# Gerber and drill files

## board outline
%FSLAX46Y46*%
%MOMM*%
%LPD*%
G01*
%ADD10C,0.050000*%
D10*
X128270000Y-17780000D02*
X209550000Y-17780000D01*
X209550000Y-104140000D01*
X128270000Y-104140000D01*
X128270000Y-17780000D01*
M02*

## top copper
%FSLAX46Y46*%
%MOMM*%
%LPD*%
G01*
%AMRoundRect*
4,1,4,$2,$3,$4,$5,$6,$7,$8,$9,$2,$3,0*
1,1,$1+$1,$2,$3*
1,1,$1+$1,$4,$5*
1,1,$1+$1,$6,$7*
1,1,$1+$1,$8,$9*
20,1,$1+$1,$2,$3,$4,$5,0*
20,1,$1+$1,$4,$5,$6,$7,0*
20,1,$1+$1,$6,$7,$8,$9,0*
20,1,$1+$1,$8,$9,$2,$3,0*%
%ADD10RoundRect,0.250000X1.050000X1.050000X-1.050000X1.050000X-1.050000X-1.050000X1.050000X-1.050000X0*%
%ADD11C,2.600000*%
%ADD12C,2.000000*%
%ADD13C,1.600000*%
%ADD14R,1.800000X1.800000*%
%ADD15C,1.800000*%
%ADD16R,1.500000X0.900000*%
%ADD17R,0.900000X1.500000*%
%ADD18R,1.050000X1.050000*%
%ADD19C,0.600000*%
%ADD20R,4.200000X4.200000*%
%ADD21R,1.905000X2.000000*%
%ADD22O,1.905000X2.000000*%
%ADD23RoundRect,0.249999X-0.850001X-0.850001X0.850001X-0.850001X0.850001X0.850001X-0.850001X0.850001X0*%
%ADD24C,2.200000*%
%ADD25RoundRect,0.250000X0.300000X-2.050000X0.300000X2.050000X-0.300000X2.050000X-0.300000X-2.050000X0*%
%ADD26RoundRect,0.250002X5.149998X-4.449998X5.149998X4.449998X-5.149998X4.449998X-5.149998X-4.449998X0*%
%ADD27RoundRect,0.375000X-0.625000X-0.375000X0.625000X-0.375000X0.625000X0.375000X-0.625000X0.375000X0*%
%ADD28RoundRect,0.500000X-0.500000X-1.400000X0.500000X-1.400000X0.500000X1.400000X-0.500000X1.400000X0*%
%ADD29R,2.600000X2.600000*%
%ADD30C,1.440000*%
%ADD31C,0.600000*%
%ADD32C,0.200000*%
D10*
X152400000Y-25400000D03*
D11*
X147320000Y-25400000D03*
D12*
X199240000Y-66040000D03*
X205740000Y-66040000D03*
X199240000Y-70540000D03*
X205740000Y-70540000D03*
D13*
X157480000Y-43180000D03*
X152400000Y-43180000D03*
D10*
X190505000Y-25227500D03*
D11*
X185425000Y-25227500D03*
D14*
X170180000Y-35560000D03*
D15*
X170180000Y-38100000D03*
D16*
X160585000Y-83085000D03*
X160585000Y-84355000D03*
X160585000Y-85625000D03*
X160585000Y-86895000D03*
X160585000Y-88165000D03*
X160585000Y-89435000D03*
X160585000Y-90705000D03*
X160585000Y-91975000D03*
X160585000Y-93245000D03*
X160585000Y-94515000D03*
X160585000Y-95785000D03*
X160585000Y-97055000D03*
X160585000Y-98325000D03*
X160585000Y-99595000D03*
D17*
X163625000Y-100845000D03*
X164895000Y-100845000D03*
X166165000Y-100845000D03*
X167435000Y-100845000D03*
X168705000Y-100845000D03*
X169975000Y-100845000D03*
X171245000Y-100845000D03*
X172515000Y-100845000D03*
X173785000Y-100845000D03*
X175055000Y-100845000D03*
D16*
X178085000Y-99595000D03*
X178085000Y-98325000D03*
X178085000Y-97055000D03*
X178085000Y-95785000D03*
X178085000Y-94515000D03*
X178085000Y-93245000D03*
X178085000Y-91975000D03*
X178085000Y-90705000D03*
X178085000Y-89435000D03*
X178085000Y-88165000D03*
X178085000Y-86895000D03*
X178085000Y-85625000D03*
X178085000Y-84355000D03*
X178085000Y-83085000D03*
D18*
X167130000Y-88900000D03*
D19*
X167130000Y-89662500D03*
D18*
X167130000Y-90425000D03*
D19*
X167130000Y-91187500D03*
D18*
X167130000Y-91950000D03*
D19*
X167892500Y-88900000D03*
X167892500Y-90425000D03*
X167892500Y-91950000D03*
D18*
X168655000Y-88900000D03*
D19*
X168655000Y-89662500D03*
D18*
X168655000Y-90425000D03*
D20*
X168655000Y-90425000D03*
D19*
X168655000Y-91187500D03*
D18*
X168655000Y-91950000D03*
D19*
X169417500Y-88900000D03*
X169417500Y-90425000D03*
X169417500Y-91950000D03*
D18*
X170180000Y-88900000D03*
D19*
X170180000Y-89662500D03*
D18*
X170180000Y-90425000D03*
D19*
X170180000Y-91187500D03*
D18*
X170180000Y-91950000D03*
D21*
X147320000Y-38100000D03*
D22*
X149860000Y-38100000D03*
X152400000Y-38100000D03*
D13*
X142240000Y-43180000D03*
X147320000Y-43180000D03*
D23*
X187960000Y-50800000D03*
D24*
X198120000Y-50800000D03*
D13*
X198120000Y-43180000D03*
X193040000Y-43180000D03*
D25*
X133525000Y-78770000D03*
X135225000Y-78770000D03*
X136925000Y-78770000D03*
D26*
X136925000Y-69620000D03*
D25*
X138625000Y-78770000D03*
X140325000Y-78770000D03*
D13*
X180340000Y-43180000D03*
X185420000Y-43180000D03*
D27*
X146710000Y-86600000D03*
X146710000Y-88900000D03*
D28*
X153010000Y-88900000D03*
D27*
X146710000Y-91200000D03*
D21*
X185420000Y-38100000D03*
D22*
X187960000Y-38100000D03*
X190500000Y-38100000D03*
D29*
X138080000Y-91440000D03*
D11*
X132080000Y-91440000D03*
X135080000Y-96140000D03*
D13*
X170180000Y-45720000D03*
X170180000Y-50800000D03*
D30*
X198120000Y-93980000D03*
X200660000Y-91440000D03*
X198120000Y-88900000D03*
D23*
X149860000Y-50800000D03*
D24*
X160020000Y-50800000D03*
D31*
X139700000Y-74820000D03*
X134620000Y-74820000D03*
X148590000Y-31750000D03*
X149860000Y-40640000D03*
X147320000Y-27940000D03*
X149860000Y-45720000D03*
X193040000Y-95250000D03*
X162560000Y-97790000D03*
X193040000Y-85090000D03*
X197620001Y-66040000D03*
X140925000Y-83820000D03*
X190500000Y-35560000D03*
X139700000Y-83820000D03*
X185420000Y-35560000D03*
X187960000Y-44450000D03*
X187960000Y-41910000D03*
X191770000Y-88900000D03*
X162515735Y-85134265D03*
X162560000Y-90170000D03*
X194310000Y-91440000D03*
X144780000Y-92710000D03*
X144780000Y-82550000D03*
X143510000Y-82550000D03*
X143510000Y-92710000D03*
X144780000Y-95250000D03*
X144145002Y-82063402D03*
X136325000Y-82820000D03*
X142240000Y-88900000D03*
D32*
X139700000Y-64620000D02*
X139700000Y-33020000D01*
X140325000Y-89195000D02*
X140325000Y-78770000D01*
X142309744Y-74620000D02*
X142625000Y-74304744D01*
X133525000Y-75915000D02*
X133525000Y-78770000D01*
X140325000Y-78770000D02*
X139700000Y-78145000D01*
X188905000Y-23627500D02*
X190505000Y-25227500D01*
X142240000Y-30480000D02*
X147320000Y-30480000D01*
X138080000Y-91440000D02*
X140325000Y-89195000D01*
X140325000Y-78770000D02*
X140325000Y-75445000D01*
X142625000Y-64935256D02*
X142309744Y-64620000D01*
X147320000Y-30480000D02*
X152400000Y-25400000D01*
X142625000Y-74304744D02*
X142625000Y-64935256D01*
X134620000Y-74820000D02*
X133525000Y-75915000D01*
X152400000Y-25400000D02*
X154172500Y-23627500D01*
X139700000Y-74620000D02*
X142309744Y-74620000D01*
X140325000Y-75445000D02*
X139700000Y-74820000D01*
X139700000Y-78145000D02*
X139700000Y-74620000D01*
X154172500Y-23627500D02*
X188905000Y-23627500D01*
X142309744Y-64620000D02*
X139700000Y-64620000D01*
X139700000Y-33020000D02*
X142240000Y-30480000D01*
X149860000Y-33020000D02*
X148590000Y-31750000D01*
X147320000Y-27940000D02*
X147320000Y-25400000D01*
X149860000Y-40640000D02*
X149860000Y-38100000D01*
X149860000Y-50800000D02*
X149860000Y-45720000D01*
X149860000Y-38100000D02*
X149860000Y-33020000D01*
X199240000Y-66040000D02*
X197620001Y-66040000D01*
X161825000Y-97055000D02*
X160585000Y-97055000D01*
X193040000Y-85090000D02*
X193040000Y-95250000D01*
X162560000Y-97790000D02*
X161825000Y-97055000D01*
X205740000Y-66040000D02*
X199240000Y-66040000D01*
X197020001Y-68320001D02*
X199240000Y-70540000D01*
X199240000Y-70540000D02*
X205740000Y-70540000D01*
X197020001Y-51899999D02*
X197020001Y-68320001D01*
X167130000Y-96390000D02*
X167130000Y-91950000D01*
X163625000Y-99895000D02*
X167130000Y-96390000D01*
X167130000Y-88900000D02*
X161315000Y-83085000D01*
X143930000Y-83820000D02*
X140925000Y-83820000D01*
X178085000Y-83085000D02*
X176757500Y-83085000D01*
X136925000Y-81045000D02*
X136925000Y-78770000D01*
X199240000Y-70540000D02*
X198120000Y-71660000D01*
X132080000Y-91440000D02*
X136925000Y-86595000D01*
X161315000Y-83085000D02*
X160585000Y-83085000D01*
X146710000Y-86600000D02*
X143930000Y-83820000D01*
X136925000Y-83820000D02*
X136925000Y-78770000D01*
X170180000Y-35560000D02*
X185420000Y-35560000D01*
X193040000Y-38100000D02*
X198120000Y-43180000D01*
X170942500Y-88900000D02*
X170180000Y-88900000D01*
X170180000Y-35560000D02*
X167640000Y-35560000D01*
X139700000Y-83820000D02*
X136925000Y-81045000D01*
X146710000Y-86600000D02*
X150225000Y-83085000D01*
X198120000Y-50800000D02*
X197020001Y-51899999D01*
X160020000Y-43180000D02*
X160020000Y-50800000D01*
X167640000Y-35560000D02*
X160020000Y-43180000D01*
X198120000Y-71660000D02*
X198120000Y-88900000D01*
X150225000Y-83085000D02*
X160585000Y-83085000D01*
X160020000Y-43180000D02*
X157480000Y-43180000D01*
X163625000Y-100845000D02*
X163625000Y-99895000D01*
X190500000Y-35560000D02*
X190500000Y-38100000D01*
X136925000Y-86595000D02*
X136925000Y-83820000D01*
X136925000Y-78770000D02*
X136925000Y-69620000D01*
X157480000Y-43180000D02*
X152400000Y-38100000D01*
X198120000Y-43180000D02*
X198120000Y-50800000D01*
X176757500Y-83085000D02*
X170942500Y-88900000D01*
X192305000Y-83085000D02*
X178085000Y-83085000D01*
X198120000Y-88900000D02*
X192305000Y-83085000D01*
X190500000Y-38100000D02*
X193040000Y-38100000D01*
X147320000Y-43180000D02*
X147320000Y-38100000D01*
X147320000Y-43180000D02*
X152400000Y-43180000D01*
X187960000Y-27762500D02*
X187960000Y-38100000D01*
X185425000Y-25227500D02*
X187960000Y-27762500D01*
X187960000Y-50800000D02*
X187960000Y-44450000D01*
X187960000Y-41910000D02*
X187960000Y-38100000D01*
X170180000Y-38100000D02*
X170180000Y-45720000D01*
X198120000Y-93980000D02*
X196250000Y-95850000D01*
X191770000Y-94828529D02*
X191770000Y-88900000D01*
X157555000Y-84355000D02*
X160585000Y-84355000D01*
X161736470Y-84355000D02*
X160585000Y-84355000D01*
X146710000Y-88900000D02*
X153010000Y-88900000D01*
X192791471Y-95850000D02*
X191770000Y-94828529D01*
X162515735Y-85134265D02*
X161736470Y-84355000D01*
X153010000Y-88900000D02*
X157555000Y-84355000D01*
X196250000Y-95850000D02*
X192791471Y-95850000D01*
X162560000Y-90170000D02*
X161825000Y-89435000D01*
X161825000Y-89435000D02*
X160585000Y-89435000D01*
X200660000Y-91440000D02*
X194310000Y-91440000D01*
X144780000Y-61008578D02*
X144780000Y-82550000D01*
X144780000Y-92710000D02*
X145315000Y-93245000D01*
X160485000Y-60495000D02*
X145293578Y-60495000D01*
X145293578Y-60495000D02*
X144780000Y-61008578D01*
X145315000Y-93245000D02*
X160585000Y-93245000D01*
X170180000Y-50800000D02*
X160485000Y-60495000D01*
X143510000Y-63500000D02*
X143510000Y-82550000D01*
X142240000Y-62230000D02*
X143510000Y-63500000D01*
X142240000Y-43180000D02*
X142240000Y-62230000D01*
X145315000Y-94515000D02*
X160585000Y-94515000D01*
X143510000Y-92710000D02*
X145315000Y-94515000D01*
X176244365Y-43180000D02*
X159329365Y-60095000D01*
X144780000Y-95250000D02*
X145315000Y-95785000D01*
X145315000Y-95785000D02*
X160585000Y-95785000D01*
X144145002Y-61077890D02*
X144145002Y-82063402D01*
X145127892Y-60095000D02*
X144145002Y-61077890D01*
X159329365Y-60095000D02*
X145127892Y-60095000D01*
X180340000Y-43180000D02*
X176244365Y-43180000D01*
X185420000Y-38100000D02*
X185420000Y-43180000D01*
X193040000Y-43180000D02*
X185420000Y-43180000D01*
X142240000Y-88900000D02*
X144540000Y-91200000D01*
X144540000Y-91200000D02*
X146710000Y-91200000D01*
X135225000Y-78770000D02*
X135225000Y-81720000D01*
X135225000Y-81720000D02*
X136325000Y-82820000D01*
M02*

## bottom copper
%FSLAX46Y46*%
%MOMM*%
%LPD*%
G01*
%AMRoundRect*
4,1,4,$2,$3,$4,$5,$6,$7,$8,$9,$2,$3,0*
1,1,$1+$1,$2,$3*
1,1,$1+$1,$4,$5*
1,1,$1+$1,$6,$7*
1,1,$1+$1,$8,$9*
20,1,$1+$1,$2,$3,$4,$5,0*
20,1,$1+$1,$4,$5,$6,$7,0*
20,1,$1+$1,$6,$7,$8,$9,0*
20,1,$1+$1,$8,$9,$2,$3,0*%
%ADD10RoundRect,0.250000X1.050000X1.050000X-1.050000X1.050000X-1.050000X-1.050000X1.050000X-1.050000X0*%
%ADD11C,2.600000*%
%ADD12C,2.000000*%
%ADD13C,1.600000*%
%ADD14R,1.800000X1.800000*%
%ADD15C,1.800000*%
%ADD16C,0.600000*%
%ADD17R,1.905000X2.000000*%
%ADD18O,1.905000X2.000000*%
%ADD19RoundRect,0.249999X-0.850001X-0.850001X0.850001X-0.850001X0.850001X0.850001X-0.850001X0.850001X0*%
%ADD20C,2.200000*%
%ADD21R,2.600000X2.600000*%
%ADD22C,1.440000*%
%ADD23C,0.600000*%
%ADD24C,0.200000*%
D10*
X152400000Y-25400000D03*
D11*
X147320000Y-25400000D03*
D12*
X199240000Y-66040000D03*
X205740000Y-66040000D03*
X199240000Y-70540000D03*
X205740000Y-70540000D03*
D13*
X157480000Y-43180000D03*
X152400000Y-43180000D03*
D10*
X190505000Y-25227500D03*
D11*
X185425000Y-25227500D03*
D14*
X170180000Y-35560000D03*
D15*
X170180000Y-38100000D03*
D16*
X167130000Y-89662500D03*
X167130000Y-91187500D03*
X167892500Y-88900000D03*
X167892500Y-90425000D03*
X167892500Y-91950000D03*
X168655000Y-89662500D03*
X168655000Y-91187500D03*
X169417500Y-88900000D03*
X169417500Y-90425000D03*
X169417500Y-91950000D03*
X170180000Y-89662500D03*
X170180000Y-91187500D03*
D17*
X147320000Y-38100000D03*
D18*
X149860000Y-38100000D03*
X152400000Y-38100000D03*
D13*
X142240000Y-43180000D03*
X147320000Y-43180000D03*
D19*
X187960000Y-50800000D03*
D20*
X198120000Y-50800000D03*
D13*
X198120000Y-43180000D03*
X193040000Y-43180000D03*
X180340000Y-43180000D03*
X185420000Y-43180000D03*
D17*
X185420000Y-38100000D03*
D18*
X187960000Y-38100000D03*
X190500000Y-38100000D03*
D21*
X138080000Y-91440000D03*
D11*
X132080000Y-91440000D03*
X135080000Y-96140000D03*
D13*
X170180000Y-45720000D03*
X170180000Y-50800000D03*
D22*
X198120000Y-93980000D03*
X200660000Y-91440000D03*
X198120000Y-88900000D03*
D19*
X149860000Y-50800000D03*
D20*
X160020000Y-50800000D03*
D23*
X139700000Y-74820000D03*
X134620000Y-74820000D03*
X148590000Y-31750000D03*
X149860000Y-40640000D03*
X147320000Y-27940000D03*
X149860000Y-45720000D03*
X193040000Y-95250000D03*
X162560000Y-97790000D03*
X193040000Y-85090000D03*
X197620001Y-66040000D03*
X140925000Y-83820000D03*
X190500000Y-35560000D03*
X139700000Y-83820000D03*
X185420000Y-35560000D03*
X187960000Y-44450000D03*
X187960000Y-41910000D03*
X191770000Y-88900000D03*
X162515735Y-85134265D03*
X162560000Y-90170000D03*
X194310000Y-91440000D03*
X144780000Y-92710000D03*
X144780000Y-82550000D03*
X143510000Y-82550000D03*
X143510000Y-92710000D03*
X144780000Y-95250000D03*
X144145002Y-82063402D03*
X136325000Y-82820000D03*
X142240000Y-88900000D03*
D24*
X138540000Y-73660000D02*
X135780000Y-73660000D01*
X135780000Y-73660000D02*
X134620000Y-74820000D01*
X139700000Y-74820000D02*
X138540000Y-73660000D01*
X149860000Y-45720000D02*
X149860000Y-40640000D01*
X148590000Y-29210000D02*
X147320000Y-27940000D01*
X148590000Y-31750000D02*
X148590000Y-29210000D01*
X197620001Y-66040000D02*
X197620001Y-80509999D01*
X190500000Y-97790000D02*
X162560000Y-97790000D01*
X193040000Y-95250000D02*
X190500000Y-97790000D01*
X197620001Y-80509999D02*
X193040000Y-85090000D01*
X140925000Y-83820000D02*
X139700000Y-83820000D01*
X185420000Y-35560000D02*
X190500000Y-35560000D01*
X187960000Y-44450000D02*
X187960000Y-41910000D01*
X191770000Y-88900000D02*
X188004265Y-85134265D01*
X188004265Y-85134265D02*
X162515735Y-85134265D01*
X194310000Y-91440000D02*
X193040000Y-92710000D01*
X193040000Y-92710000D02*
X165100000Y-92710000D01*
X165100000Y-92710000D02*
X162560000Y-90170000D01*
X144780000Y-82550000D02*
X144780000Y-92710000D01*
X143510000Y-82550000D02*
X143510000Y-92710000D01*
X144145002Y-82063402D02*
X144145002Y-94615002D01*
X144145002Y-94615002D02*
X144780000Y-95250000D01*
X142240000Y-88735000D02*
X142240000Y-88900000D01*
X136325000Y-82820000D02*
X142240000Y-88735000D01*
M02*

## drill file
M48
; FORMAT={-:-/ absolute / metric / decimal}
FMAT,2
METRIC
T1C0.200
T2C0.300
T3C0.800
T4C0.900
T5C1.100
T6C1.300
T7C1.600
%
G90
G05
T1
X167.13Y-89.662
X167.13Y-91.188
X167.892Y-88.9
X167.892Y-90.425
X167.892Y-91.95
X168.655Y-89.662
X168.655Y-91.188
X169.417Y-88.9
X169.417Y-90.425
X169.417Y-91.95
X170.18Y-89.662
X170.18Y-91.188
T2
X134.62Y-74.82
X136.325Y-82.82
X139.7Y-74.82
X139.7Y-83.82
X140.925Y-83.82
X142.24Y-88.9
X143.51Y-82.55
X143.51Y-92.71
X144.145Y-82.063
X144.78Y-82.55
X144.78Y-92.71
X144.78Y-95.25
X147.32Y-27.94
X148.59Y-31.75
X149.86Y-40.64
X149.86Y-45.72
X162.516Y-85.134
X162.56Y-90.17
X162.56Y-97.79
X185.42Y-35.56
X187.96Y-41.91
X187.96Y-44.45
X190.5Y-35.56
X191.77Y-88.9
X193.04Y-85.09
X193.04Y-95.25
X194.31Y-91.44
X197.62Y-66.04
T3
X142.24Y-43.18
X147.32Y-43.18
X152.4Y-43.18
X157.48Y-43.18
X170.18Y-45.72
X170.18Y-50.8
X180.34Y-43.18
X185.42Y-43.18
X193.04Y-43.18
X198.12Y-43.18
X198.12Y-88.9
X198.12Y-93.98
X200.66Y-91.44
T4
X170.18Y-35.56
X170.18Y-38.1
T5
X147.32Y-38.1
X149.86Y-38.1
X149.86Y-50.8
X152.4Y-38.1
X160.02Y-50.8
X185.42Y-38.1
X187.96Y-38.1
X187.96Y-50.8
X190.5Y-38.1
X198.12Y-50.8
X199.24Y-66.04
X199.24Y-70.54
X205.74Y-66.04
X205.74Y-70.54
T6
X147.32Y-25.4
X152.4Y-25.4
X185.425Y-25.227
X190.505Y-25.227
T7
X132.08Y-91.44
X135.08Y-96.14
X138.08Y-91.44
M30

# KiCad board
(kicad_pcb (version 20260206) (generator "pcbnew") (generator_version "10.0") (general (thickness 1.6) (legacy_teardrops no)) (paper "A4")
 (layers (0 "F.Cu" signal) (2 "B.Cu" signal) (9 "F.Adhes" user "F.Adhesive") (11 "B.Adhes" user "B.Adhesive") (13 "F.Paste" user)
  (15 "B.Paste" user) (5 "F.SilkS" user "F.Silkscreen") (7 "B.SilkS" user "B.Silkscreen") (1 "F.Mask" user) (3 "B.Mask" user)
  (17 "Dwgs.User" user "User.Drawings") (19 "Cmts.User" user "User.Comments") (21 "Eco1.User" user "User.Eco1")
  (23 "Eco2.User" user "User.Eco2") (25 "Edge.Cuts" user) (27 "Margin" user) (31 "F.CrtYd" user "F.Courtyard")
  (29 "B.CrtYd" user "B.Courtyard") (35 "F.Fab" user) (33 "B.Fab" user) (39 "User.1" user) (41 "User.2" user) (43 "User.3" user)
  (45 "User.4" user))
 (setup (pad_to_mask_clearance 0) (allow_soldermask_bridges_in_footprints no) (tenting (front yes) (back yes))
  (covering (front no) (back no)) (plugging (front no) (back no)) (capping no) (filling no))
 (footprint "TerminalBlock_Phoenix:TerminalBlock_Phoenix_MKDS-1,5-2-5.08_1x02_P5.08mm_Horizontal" (layer "F.Cu") (at 152.4 25.4 180)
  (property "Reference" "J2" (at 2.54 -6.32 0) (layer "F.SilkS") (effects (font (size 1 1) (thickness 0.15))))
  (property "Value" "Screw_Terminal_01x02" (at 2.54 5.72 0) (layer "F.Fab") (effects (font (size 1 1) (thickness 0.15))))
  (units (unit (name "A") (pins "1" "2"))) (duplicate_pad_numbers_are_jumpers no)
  (pad "1" thru_hole roundrect (at 0 0 180) (size 2.6 2.6) (drill 1.3) (layers "*.Cu" "*.Mask") (remove_unused_layers no)
   (roundrect_rratio 0.096154) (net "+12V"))
  (pad "2" thru_hole circle (at 5.08 0 180) (size 2.6 2.6) (drill 1.3) (layers "*.Cu" "*.Mask") (remove_unused_layers no) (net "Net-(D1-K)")))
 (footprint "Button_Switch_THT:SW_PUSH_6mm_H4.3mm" (layer "F.Cu") (at 199.24 66.04)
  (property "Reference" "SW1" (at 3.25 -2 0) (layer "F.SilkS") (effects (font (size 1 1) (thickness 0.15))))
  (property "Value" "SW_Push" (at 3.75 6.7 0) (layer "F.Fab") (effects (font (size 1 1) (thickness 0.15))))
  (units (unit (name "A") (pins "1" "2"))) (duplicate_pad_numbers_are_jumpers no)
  (pad "1" thru_hole circle (at 0 0 90) (size 2 2) (drill 1.1) (layers "*.Cu" "*.Mask") (remove_unused_layers no) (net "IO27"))
  (pad "1" thru_hole circle (at 6.5 0 90) (size 2 2) (drill 1.1) (layers "*.Cu" "*.Mask") (remove_unused_layers no) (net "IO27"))
  (pad "2" thru_hole circle (at 0 4.5 90) (size 2 2) (drill 1.1) (layers "*.Cu" "*.Mask") (remove_unused_layers no) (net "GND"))
  (pad "2" thru_hole circle (at 6.5 4.5 90) (size 2 2) (drill 1.1) (layers "*.Cu" "*.Mask") (remove_unused_layers no) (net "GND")))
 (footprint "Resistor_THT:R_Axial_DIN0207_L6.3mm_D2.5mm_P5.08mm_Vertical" (layer "F.Cu") (at 157.48 43.18 180)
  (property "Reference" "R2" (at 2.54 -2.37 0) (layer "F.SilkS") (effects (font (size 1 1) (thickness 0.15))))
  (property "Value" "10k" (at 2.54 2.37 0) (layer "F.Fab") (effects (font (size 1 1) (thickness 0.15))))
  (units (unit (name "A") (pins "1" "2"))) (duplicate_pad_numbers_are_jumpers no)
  (pad "1" thru_hole circle (at 0 0 180) (size 1.6 1.6) (drill 0.8) (layers "*.Cu" "*.Mask") (remove_unused_layers no) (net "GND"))
  (pad "2" thru_hole circle (at 5.08 0 180) (size 1.6 1.6) (drill 0.8) (layers "*.Cu" "*.Mask") (remove_unused_layers no) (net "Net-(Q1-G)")))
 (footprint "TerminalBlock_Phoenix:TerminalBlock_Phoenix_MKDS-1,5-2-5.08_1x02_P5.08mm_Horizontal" (layer "F.Cu") (at 190.505 25.2275 180)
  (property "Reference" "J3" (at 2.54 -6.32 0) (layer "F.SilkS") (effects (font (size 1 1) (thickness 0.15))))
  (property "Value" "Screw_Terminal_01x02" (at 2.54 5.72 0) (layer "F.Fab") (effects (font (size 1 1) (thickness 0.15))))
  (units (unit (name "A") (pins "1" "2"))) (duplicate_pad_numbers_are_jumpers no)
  (pad "1" thru_hole roundrect (at 0 0 180) (size 2.6 2.6) (drill 1.3) (layers "*.Cu" "*.Mask") (remove_unused_layers no)
   (roundrect_rratio 0.096154) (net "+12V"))
  (pad "2" thru_hole circle (at 5.08 0 180) (size 2.6 2.6) (drill 1.3) (layers "*.Cu" "*.Mask") (remove_unused_layers no) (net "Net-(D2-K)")))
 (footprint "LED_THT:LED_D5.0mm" (layer "F.Cu") (at 170.18 35.56 -90)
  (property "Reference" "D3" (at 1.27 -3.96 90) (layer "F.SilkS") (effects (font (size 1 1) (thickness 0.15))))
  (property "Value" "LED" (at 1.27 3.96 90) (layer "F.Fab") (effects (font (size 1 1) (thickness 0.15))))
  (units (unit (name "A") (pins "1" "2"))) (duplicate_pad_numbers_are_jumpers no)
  (pad "1" thru_hole rect (at 0 0 270) (size 1.8 1.8) (drill 0.9) (layers "*.Cu" "*.Mask") (remove_unused_layers no) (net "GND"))
  (pad "2" thru_hole circle (at 2.54 0 270) (size 1.8 1.8) (drill 0.9) (layers "*.Cu" "*.Mask") (remove_unused_layers no) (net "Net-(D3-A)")))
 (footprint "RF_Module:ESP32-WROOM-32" (layer "F.Cu") (at 169.335 91.335)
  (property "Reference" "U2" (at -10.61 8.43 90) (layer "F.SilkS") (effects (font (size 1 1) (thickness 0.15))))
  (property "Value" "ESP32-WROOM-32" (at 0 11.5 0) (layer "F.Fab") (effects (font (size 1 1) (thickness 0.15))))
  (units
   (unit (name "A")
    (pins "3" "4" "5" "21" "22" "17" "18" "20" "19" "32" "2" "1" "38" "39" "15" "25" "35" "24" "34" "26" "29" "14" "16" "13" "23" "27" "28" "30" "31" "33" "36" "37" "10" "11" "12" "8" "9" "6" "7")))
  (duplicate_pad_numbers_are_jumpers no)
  (pad "1" smd rect (at -8.75 -8.25) (size 1.5 0.9) (layers "F.Cu" "F.Mask" "F.Paste") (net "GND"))
  (pad "2" smd rect (at -8.75 -6.98) (size 1.5 0.9) (layers "F.Cu" "F.Mask" "F.Paste") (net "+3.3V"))
  (pad "3" smd rect (at -8.75 -5.71) (size 1.5 0.9) (layers "F.Cu" "F.Mask" "F.Paste") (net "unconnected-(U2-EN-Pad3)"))
  (pad "4" smd rect (at -8.75 -4.44) (size 1.5 0.9) (layers "F.Cu" "F.Mask" "F.Paste") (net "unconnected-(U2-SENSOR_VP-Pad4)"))
  (pad "5" smd rect (at -8.75 -3.17) (size 1.5 0.9) (layers "F.Cu" "F.Mask" "F.Paste") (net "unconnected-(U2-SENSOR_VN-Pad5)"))
  (pad "6" smd rect (at -8.75 -1.9) (size 1.5 0.9) (layers "F.Cu" "F.Mask" "F.Paste") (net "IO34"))
  (pad "7" smd rect (at -8.75 -0.63) (size 1.5 0.9) (layers "F.Cu" "F.Mask" "F.Paste") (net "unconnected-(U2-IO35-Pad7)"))
  (pad "8" smd rect (at -8.75 0.64) (size 1.5 0.9) (layers "F.Cu" "F.Mask" "F.Paste") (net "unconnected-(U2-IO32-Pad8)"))
  (pad "9" smd rect (at -8.75 1.91) (size 1.5 0.9) (layers "F.Cu" "F.Mask" "F.Paste") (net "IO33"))
  (pad "10" smd rect (at -8.75 3.18) (size 1.5 0.9) (layers "F.Cu" "F.Mask" "F.Paste") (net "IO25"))
  (pad "11" smd rect (at -8.75 4.45) (size 1.5 0.9) (layers "F.Cu" "F.Mask" "F.Paste") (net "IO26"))
  (pad "12" smd rect (at -8.75 5.72) (size 1.5 0.9) (layers "F.Cu" "F.Mask" "F.Paste") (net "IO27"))
  (pad "13" smd rect (at -8.75 6.99) (size 1.5 0.9) (layers "F.Cu" "F.Mask" "F.Paste") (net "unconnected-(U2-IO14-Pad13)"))
  (pad "14" smd rect (at -8.75 8.26) (size 1.5 0.9) (layers "F.Cu" "F.Mask" "F.Paste") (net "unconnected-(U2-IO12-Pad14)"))
  (pad "15" smd rect (at -5.71 9.51 90) (size 1.5 0.9) (layers "F.Cu" "F.Mask" "F.Paste") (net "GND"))
  (pad "16" smd rect (at -4.44 9.51 90) (size 1.5 0.9) (layers "F.Cu" "F.Mask" "F.Paste") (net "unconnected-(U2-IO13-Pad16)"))
  (pad "17" smd rect (at -3.17 9.51 90) (size 1.5 0.9) (layers "F.Cu" "F.Mask" "F.Paste") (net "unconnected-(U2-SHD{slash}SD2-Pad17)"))
  (pad "18" smd rect (at -1.9 9.51 90) (size 1.5 0.9) (layers "F.Cu" "F.Mask" "F.Paste") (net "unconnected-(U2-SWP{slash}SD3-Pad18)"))
  (pad "19" smd rect (at -0.63 9.51 90) (size 1.5 0.9) (layers "F.Cu" "F.Mask" "F.Paste") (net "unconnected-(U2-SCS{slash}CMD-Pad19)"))
  (pad "20" smd rect (at 0.64 9.51 90) (size 1.5 0.9) (layers "F.Cu" "F.Mask" "F.Paste") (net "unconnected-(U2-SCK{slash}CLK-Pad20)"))
  (pad "21" smd rect (at 1.91 9.51 90) (size 1.5 0.9) (layers "F.Cu" "F.Mask" "F.Paste") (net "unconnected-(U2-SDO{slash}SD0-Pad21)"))
  (pad "22" smd rect (at 3.18 9.51 90) (size 1.5 0.9) (layers "F.Cu" "F.Mask" "F.Paste") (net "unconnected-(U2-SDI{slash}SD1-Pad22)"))
  (pad "23" smd rect (at 4.45 9.51 90) (size 1.5 0.9) (layers "F.Cu" "F.Mask" "F.Paste") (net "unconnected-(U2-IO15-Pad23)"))
  (pad "24" smd rect (at 5.72 9.51 90) (size 1.5 0.9) (layers "F.Cu" "F.Mask" "F.Paste") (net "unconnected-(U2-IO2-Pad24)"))
  (pad "25" smd rect (at 8.75 8.26) (size 1.5 0.9) (layers "F.Cu" "F.Mask" "F.Paste") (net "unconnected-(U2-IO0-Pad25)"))
  (pad "26" smd rect (at 8.75 6.99) (size 1.5 0.9) (layers "F.Cu" "F.Mask" "F.Paste") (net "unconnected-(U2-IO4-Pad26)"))
  (pad "27" smd rect (at 8.75 5.72) (size 1.5 0.9) (layers "F.Cu" "F.Mask" "F.Paste") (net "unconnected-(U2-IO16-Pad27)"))
  (pad "28" smd rect (at 8.75 4.45) (size 1.5 0.9) (layers "F.Cu" "F.Mask" "F.Paste") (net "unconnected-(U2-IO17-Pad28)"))
  (pad "29" smd rect (at 8.75 3.18) (size 1.5 0.9) (layers "F.Cu" "F.Mask" "F.Paste") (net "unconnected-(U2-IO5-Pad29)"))
  (pad "30" smd rect (at 8.75 1.91) (size 1.5 0.9) (layers "F.Cu" "F.Mask" "F.Paste") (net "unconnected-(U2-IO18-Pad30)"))
  (pad "31" smd rect (at 8.75 0.64) (size 1.5 0.9) (layers "F.Cu" "F.Mask" "F.Paste") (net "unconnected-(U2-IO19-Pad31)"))
  (pad "32" smd rect (at 8.75 -0.63) (size 1.5 0.9) (layers "F.Cu" "F.Mask" "F.Paste") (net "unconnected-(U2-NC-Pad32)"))
  (pad "33" smd rect (at 8.75 -1.9) (size 1.5 0.9) (layers "F.Cu" "F.Mask" "F.Paste") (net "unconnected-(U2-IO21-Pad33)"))
  (pad "34" smd rect (at 8.75 -3.17) (size 1.5 0.9) (layers "F.Cu" "F.Mask" "F.Paste") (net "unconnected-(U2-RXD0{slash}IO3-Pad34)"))
  (pad "35" smd rect (at 8.75 -4.44) (size 1.5 0.9) (layers "F.Cu" "F.Mask" "F.Paste") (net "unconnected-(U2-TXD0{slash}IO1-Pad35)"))
  (pad "36" smd rect (at 8.75 -5.71) (size 1.5 0.9) (layers "F.Cu" "F.Mask" "F.Paste") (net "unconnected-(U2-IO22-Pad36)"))
  (pad "37" smd rect (at 8.75 -6.98) (size 1.5 0.9) (layers "F.Cu" "F.Mask" "F.Paste") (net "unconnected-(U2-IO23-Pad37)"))
  (pad "38" smd rect (at 8.75 -8.25) (size 1.5 0.9) (layers "F.Cu" "F.Mask" "F.Paste") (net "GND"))
  (pad "39" smd rect (at -2.205 -2.435) (size 1.05 1.05) (layers "F.Cu" "F.Paste") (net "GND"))
  (pad "39" thru_hole circle (at -2.205 -1.6725) (size 0.6 0.6) (drill 0.2) (layers "*.Cu" "F.Mask") (remove_unused_layers no) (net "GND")
   (zone_connect 2))
  (pad "39" smd rect (at -2.205 -0.91) (size 1.05 1.05) (layers "F.Cu" "F.Paste") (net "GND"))
  (pad "39" thru_hole circle (at -2.205 -0.1475) (size 0.6 0.6) (drill 0.2) (layers "*.Cu" "F.Mask") (remove_unused_layers no) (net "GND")
   (zone_connect 2))
  (pad "39" smd rect (at -2.205 0.615) (size 1.05 1.05) (layers "F.Cu" "F.Paste") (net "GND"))
  (pad "39" thru_hole circle (at -1.4425 -2.435) (size 0.6 0.6) (drill 0.2) (layers "*.Cu" "F.Mask") (remove_unused_layers no) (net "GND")
   (zone_connect 2))
  (pad "39" thru_hole circle (at -1.4425 -0.91) (size 0.6 0.6) (drill 0.2) (layers "*.Cu" "F.Mask") (remove_unused_layers no) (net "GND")
   (zone_connect 2))
  (pad "39" thru_hole circle (at -1.4425 0.615) (size 0.6 0.6) (drill 0.2) (layers "*.Cu" "F.Mask") (remove_unused_layers no) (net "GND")
   (zone_connect 2))
  (pad "39" smd rect (at -0.68 -2.435) (size 1.05 1.05) (layers "F.Cu" "F.Paste") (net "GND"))
  (pad "39" thru_hole circle (at -0.68 -1.6725) (size 0.6 0.6) (drill 0.2) (layers "*.Cu" "F.Mask") (remove_unused_layers no) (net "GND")
   (zone_connect 2))
  (pad "39" smd rect (at -0.68 -0.91) (size 1.05 1.05) (layers "F.Cu" "F.Paste") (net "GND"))
  (pad "39" smd rect (at -0.68 -0.91) (size 4.2 4.2) (layers "F.Cu" "F.Mask") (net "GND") (zone_connect 2))
  (pad "39" thru_hole circle (at -0.68 -0.1475) (size 0.6 0.6) (drill 0.2) (layers "*.Cu" "F.Mask") (remove_unused_layers no) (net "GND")
   (zone_connect 2))
  (pad "39" smd rect (at -0.68 0.615) (size 1.05 1.05) (layers "F.Cu" "F.Paste") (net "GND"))
  (pad "39" thru_hole circle (at 0.0825 -2.435) (size 0.6 0.6) (drill 0.2) (layers "*.Cu" "F.Mask") (remove_unused_layers no) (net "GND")
   (zone_connect 2))
  (pad "39" thru_hole circle (at 0.0825 -0.91) (size 0.6 0.6) (drill 0.2) (layers "*.Cu" "F.Mask") (remove_unused_layers no) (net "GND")
   (zone_connect 2))
  (pad "39" thru_hole circle (at 0.0825 0.615) (size 0.6 0.6) (drill 0.2) (layers "*.Cu" "F.Mask") (remove_unused_layers no) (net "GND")
   (zone_connect 2))
  (pad "39" smd rect (at 0.845 -2.435) (size 1.05 1.05) (layers "F.Cu" "F.Paste") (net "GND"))
  (pad "39" thru_hole circle (at 0.845 -1.6725) (size 0.6 0.6) (drill 0.2) (layers "*.Cu" "F.Mask") (remove_unused_layers no) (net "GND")
   (zone_connect 2))
  (pad "39" smd rect (at 0.845 -0.91) (size 1.05 1.05) (layers "F.Cu" "F.Paste") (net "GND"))
  (pad "39" thru_hole circle (at 0.845 -0.1475) (size 0.6 0.6) (drill 0.2) (layers "*.Cu" "F.Mask") (remove_unused_layers no) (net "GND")
   (zone_connect 2))
  (pad "39" smd rect (at 0.845 0.615) (size 1.05 1.05) (layers "F.Cu" "F.Paste") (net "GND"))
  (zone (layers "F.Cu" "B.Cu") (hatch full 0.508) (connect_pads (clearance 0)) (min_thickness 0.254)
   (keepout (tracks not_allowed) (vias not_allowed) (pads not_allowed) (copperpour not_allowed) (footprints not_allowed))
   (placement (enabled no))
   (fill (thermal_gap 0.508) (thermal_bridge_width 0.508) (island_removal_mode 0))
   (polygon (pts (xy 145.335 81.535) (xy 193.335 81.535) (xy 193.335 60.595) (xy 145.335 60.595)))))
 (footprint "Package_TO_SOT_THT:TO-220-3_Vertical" (layer "F.Cu") (at 147.32 38.1)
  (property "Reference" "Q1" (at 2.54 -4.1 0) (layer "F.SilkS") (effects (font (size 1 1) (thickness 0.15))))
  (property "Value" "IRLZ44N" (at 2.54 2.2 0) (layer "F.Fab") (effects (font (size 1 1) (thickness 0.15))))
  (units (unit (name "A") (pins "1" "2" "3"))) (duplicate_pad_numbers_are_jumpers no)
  (pad "1" thru_hole rect (at 0 0) (size 1.905 2) (drill 1.1) (layers "*.Cu" "*.Mask") (remove_unused_layers no) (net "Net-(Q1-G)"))
  (pad "2" thru_hole oval (at 2.54 0) (size 1.905 2) (drill 1.1) (layers "*.Cu" "*.Mask") (remove_unused_layers no) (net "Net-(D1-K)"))
  (pad "3" thru_hole oval (at 5.08 0) (size 1.905 2) (drill 1.1) (layers "*.Cu" "*.Mask") (remove_unused_layers no) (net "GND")))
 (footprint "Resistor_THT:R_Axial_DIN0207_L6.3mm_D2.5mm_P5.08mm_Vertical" (layer "F.Cu") (at 142.24 43.18)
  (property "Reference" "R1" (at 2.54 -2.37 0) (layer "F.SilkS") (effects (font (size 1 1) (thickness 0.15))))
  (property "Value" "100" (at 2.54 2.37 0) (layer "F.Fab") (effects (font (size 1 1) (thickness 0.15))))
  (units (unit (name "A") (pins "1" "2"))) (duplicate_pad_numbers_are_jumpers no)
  (pad "1" thru_hole circle (at 0 0) (size 1.6 1.6) (drill 0.8) (layers "*.Cu" "*.Mask") (remove_unused_layers no) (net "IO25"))
  (pad "2" thru_hole circle (at 5.08 0) (size 1.6 1.6) (drill 0.8) (layers "*.Cu" "*.Mask") (remove_unused_layers no) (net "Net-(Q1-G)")))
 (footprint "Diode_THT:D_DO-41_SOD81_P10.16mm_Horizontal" (layer "F.Cu") (at 187.96 50.8)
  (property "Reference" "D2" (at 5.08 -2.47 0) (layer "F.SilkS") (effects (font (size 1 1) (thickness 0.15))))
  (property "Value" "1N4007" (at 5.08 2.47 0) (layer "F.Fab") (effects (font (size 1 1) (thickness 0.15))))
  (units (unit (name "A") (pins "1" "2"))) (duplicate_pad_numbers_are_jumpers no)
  (pad "1" thru_hole roundrect (at 0 0) (size 2.2 2.2) (drill 1.1) (layers "*.Cu" "*.Mask") (remove_unused_layers no)
   (roundrect_rratio 0.113636) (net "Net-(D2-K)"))
  (pad "2" thru_hole circle (at 10.16 0) (size 2.2 2.2) (drill 1.1) (layers "*.Cu" "*.Mask") (remove_unused_layers no) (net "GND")))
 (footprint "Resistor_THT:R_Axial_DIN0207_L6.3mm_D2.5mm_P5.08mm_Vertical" (layer "F.Cu") (at 198.12 43.18 180)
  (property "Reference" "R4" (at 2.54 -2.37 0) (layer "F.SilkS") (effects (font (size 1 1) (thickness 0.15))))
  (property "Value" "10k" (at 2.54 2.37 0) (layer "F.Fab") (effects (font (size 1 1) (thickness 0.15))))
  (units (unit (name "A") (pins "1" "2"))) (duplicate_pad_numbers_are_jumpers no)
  (pad "1" thru_hole circle (at 0 0 180) (size 1.6 1.6) (drill 0.8) (layers "*.Cu" "*.Mask") (remove_unused_layers no) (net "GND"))
  (pad "2" thru_hole circle (at 5.08 0 180) (size 1.6 1.6) (drill 0.8) (layers "*.Cu" "*.Mask") (remove_unused_layers no) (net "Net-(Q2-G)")))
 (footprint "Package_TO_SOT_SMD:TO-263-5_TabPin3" (layer "F.Cu") (at 136.925 71.12 90)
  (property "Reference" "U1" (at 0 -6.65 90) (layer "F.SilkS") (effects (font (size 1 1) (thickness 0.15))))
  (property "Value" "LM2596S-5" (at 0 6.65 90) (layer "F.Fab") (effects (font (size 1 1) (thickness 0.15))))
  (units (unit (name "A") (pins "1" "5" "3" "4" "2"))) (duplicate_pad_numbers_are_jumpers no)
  (pad "" smd roundrect (at -0.925 -2.775 90) (size 4.55 5.25) (layers "F.Paste") (roundrect_rratio 0.054945))
  (pad "" smd roundrect (at -0.925 2.775 90) (size 4.55 5.25) (layers "F.Paste") (roundrect_rratio 0.054945))
  (pad "" smd roundrect (at 3.925 -2.775 90) (size 4.55 5.25) (layers "F.Paste") (roundrect_rratio 0.054945))
  (pad "" smd roundrect (at 3.925 2.775 90) (size 4.55 5.25) (layers "F.Paste") (roundrect_rratio 0.054945))
  (pad "1" smd roundrect (at -7.65 -3.4 90) (size 4.6 1.1) (layers "F.Cu" "F.Mask" "F.Paste") (roundrect_rratio 0.227273) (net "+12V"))
  (pad "2" smd roundrect (at -7.65 -1.7 90) (size 4.6 1.1) (layers "F.Cu" "F.Mask" "F.Paste") (roundrect_rratio 0.227273) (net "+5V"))
  (pad "3" smd roundrect (at -7.65 0 90) (size 4.6 1.1) (layers "F.Cu" "F.Mask" "F.Paste") (roundrect_rratio 0.227273) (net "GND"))
  (pad "3" smd roundrect (at 1.5 0 90) (size 9.4 10.8) (layers "F.Cu" "F.Mask") (roundrect_rratio 0.026596) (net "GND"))
  (pad "4" smd roundrect (at -7.65 1.7 90) (size 4.6 1.1) (layers "F.Cu" "F.Mask" "F.Paste") (roundrect_rratio 0.227273)
   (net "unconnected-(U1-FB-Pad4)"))
  (pad "5" smd roundrect (at -7.65 3.4 90) (size 4.6 1.1) (layers "F.Cu" "F.Mask" "F.Paste") (roundrect_rratio 0.227273) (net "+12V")))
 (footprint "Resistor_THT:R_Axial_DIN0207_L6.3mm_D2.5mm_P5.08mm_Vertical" (layer "F.Cu") (at 180.34 43.18)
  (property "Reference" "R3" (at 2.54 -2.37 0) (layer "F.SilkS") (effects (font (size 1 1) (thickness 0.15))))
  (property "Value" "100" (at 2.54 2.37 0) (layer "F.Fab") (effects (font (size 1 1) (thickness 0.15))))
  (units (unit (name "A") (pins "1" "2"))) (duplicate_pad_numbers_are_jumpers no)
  (pad "1" thru_hole circle (at 0 0) (size 1.6 1.6) (drill 0.8) (layers "*.Cu" "*.Mask") (remove_unused_layers no) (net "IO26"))
  (pad "2" thru_hole circle (at 5.08 0) (size 1.6 1.6) (drill 0.8) (layers "*.Cu" "*.Mask") (remove_unused_layers no) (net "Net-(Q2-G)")))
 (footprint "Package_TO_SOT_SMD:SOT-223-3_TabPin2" (layer "F.Cu") (at 149.86 88.9)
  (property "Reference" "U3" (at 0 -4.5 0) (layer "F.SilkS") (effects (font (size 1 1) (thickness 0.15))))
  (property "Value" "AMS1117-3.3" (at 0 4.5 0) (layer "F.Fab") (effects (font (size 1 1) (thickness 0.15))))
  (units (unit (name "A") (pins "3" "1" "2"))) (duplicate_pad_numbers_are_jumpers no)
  (pad "1" smd roundrect (at -3.15 -2.3) (size 2 1.5) (layers "F.Cu" "F.Mask" "F.Paste") (roundrect_rratio 0.25) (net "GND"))
  (pad "2" smd roundrect (at -3.15 0) (size 2 1.5) (layers "F.Cu" "F.Mask" "F.Paste") (roundrect_rratio 0.25) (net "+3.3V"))
  (pad "2" smd roundrect (at 3.15 0) (size 2 3.8) (layers "F.Cu" "F.Mask" "F.Paste") (roundrect_rratio 0.25) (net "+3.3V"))
  (pad "3" smd roundrect (at -3.15 2.3) (size 2 1.5) (layers "F.Cu" "F.Mask" "F.Paste") (roundrect_rratio 0.25) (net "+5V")))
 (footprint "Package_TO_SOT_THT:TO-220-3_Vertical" (layer "F.Cu") (at 185.42 38.1)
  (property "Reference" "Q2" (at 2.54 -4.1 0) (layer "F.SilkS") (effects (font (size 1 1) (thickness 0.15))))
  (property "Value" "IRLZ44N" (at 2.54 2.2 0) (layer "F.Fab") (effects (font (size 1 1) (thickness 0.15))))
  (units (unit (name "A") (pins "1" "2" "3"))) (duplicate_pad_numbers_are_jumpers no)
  (pad "1" thru_hole rect (at 0 0) (size 1.905 2) (drill 1.1) (layers "*.Cu" "*.Mask") (remove_unused_layers no) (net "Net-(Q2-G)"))
  (pad "2" thru_hole oval (at 2.54 0) (size 1.905 2) (drill 1.1) (layers "*.Cu" "*.Mask") (remove_unused_layers no) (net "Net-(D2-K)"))
  (pad "3" thru_hole oval (at 5.08 0) (size 1.905 2) (drill 1.1) (layers "*.Cu" "*.Mask") (remove_unused_layers no) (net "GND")))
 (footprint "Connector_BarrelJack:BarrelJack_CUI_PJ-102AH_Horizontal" (layer "F.Cu") (at 138.08 91.44 -90)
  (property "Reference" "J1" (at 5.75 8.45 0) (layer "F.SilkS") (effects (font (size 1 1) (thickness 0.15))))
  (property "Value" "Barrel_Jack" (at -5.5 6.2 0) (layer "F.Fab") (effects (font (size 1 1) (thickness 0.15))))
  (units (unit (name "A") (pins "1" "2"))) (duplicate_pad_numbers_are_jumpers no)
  (pad "1" thru_hole rect (at 0 0 270) (size 2.6 2.6) (drill 1.6) (layers "*.Cu" "*.Mask") (remove_unused_layers no) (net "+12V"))
  (pad "2" thru_hole circle (at 0 6 270) (size 2.6 2.6) (drill 1.6) (layers "*.Cu" "*.Mask") (remove_unused_layers no) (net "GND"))
  (pad "3" thru_hole circle (at 4.7 3 270) (size 2.6 2.6) (drill 1.6) (layers "*.Cu" "*.Mask") (remove_unused_layers no)))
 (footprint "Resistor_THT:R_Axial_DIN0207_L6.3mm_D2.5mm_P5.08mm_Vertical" (layer "F.Cu") (at 170.18 45.72 -90)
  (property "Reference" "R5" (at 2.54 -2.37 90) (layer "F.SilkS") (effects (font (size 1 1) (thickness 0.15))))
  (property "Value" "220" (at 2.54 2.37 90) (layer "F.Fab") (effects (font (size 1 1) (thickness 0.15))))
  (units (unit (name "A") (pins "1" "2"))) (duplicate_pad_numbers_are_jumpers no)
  (pad "1" thru_hole circle (at 0 0 270) (size 1.6 1.6) (drill 0.8) (layers "*.Cu" "*.Mask") (remove_unused_layers no) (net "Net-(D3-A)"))
  (pad "2" thru_hole circle (at 5.08 0 270) (size 1.6 1.6) (drill 0.8) (layers "*.Cu" "*.Mask") (remove_unused_layers no) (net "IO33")))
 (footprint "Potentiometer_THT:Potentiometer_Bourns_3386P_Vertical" (layer "F.Cu") (at 198.12 93.98)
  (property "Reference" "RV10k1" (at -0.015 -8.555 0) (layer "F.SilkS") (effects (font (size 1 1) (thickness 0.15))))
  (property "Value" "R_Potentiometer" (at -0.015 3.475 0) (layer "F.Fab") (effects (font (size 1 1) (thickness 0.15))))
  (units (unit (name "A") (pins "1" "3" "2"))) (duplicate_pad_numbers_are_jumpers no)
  (pad "1" thru_hole circle (at 0 0) (size 1.44 1.44) (drill 0.8) (layers "*.Cu" "*.Mask") (remove_unused_layers no) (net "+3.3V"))
  (pad "2" thru_hole circle (at 2.54 -2.54) (size 1.44 1.44) (drill 0.8) (layers "*.Cu" "*.Mask") (remove_unused_layers no) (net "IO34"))
  (pad "3" thru_hole circle (at 0 -5.08) (size 1.44 1.44) (drill 0.8) (layers "*.Cu" "*.Mask") (remove_unused_layers no) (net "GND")))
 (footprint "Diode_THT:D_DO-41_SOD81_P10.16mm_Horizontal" (layer "F.Cu") (at 149.86 50.8)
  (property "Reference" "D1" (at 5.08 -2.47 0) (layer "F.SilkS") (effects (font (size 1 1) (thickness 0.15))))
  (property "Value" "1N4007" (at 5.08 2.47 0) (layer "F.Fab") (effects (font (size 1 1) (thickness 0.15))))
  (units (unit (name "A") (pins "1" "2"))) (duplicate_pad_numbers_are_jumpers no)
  (pad "1" thru_hole roundrect (at 0 0) (size 2.2 2.2) (drill 1.1) (layers "*.Cu" "*.Mask") (remove_unused_layers no)
   (roundrect_rratio 0.113636) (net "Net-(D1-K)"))
  (pad "2" thru_hole circle (at 10.16 0) (size 2.2 2.2) (drill 1.1) (layers "*.Cu" "*.Mask") (remove_unused_layers no) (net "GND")))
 (gr_rect (start 128.27 17.78) (end 209.55 104.14) (stroke (width 0.05) (type default)) (fill no) (layer "Edge.Cuts"))
 (segment (start 139.7 64.62) (end 139.7 33.02) (width 0.2) (layer "F.Cu") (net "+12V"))
 (segment (start 140.325 89.195) (end 140.325 78.77) (width 0.2) (layer "F.Cu") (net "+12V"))
 (segment (start 142.309744 74.62) (end 142.625 74.304744) (width 0.2) (layer "F.Cu") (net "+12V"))
 (segment (start 133.525 75.915) (end 133.525 78.77) (width 0.2) (layer "F.Cu") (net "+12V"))
 (segment (start 140.325 78.77) (end 139.7 78.145) (width 0.2) (layer "F.Cu") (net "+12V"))
 (segment (start 188.905 23.6275) (end 190.505 25.2275) (width 0.2) (layer "F.Cu") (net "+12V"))
 (segment (start 142.24 30.48) (end 147.32 30.48) (width 0.2) (layer "F.Cu") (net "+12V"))
 (segment (start 138.08 91.44) (end 140.325 89.195) (width 0.2) (layer "F.Cu") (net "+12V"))
 (segment (start 140.325 78.77) (end 140.325 75.445) (width 0.2) (layer "F.Cu") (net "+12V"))
 (segment (start 142.625 64.935256) (end 142.309744 64.62) (width 0.2) (layer "F.Cu") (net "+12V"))
 (segment (start 147.32 30.48) (end 152.4 25.4) (width 0.2) (layer "F.Cu") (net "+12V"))
 (segment (start 142.625 74.304744) (end 142.625 64.935256) (width 0.2) (layer "F.Cu") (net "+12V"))
 (segment (start 134.62 74.82) (end 133.525 75.915) (width 0.2) (layer "F.Cu") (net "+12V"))
 (segment (start 152.4 25.4) (end 154.1725 23.6275) (width 0.2) (layer "F.Cu") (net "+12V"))
 (segment (start 139.7 74.62) (end 142.309744 74.62) (width 0.2) (layer "F.Cu") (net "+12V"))
 (segment (start 140.325 75.445) (end 139.7 74.82) (width 0.2) (layer "F.Cu") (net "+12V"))
 (segment (start 139.7 78.145) (end 139.7 74.62) (width 0.2) (layer "F.Cu") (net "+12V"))
 (segment (start 154.1725 23.6275) (end 188.905 23.6275) (width 0.2) (layer "F.Cu") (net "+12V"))
 (segment (start 142.309744 64.62) (end 139.7 64.62) (width 0.2) (layer "F.Cu") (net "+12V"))
 (segment (start 139.7 33.02) (end 142.24 30.48) (width 0.2) (layer "F.Cu") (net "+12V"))
 (via (at 139.7 74.82) (size 0.6) (drill 0.3) (layers "F.Cu" "B.Cu") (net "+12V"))
 (via (at 134.62 74.82) (size 0.6) (drill 0.3) (layers "F.Cu" "B.Cu") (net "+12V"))
 (segment (start 138.54 73.66) (end 135.78 73.66) (width 0.2) (layer "B.Cu") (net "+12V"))
 (segment (start 135.78 73.66) (end 134.62 74.82) (width 0.2) (layer "B.Cu") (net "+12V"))
 (segment (start 139.7 74.82) (end 138.54 73.66) (width 0.2) (layer "B.Cu") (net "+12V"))
 (segment (start 149.86 33.02) (end 148.59 31.75) (width 0.2) (layer "F.Cu") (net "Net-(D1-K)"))
 (segment (start 147.32 27.94) (end 147.32 25.4) (width 0.2) (layer "F.Cu") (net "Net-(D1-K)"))
 (segment (start 149.86 40.64) (end 149.86 38.1) (width 0.2) (layer "F.Cu") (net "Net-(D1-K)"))
 (segment (start 149.86 50.8) (end 149.86 45.72) (width 0.2) (layer "F.Cu") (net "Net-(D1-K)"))
 (segment (start 149.86 38.1) (end 149.86 33.02) (width 0.2) (layer "F.Cu") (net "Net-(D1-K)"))
 (via (at 148.59 31.75) (size 0.6) (drill 0.3) (layers "F.Cu" "B.Cu") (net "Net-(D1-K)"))
 (via (at 149.86 40.64) (size 0.6) (drill 0.3) (layers "F.Cu" "B.Cu") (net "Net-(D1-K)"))
 (via (at 147.32 27.94) (size 0.6) (drill 0.3) (layers "F.Cu" "B.Cu") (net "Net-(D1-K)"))
 (via (at 149.86 45.72) (size 0.6) (drill 0.3) (layers "F.Cu" "B.Cu") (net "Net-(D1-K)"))
 (segment (start 149.86 45.72) (end 149.86 40.64) (width 0.2) (layer "B.Cu") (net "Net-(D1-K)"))
 (segment (start 148.59 29.21) (end 147.32 27.94) (width 0.2) (layer "B.Cu") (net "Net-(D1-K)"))
 (segment (start 148.59 31.75) (end 148.59 29.21) (width 0.2) (layer "B.Cu") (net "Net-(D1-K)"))
 (segment (start 199.24 66.04) (end 197.620001 66.04) (width 0.2) (layer "F.Cu") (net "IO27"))
 (segment (start 161.825 97.055) (end 160.585 97.055) (width 0.2) (layer "F.Cu") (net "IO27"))
 (segment (start 193.04 85.09) (end 193.04 95.25) (width 0.2) (layer "F.Cu") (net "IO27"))
 (segment (start 162.56 97.79) (end 161.825 97.055) (width 0.2) (layer "F.Cu") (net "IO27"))
 (segment (start 205.74 66.04) (end 199.24 66.04) (width 0.2) (layer "F.Cu") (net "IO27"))
 (via (at 193.04 95.25) (size 0.6) (drill 0.3) (layers "F.Cu" "B.Cu") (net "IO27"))
 (via (at 162.56 97.79) (size 0.6) (drill 0.3) (layers "F.Cu" "B.Cu") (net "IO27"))
 (via (at 193.04 85.09) (size 0.6) (drill 0.3) (layers "F.Cu" "B.Cu") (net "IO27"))
 (via (at 197.620001 66.04) (size 0.6) (drill 0.3) (layers "F.Cu" "B.Cu") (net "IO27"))
 (segment (start 197.620001 66.04) (end 197.620001 80.509999) (width 0.2) (layer "B.Cu") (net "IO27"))
 (segment (start 190.5 97.79) (end 162.56 97.79) (width 0.2) (layer "B.Cu") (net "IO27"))
 (segment (start 193.04 95.25) (end 190.5 97.79) (width 0.2) (layer "B.Cu") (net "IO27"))
 (segment (start 197.620001 80.509999) (end 193.04 85.09) (width 0.2) (layer "B.Cu") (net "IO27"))
 (segment (start 197.020001 68.320001) (end 199.24 70.54) (width 0.2) (layer "F.Cu") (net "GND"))
 (segment (start 199.24 70.54) (end 205.74 70.54) (width 0.2) (layer "F.Cu") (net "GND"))
 (segment (start 197.020001 51.899999) (end 197.020001 68.320001) (width 0.2) (layer "F.Cu") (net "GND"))
 (segment (start 167.13 96.39) (end 167.13 91.95) (width 0.2) (layer "F.Cu") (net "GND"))
 (segment (start 163.625 99.895) (end 167.13 96.39) (width 0.2) (layer "F.Cu") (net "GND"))
 (segment (start 167.13 88.9) (end 161.315 83.085) (width 0.2) (layer "F.Cu") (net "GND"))
 (segment (start 143.93 83.82) (end 140.925 83.82) (width 0.2) (layer "F.Cu") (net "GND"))
 (segment (start 178.085 83.085) (end 176.7575 83.085) (width 0.2) (layer "F.Cu") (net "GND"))
 (segment (start 136.925 81.045) (end 136.925 78.77) (width 0.2) (layer "F.Cu") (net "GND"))
 (segment (start 199.24 70.54) (end 198.12 71.66) (width 0.2) (layer "F.Cu") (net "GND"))
 (segment (start 132.08 91.44) (end 136.925 86.595) (width 0.2) (layer "F.Cu") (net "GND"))
 (segment (start 161.315 83.085) (end 160.585 83.085) (width 0.2) (layer "F.Cu") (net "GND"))
 (segment (start 146.71 86.6) (end 143.93 83.82) (width 0.2) (layer "F.Cu") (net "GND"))
 (segment (start 136.925 83.82) (end 136.925 78.77) (width 0.2) (layer "F.Cu") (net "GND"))
 (segment (start 170.18 35.56) (end 185.42 35.56) (width 0.2) (layer "F.Cu") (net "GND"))
 (segment (start 193.04 38.1) (end 198.12 43.18) (width 0.2) (layer "F.Cu") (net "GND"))
 (segment (start 170.9425 88.9) (end 170.18 88.9) (width 0.2) (layer "F.Cu") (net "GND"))
 (segment (start 170.18 35.56) (end 167.64 35.56) (width 0.2) (layer "F.Cu") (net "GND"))
 (segment (start 139.7 83.82) (end 136.925 81.045) (width 0.2) (layer "F.Cu") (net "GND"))
 (segment (start 146.71 86.6) (end 150.225 83.085) (width 0.2) (layer "F.Cu") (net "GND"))
 (segment (start 198.12 50.8) (end 197.020001 51.899999) (width 0.2) (layer "F.Cu") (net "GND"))
 (segment (start 160.02 43.18) (end 160.02 50.8) (width 0.2) (layer "F.Cu") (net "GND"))
 (segment (start 167.64 35.56) (end 160.02 43.18) (width 0.2) (layer "F.Cu") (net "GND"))
 (segment (start 198.12 71.66) (end 198.12 88.9) (width 0.2) (layer "F.Cu") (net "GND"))
 (segment (start 150.225 83.085) (end 160.585 83.085) (width 0.2) (layer "F.Cu") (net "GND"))
 (segment (start 160.02 43.18) (end 157.48 43.18) (width 0.2) (layer "F.Cu") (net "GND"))
 (segment (start 163.625 100.845) (end 163.625 99.895) (width 0.2) (layer "F.Cu") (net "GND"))
 (segment (start 190.5 35.56) (end 190.5 38.1) (width 0.2) (layer "F.Cu") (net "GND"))
 (segment (start 136.925 86.595) (end 136.925 83.82) (width 0.2) (layer "F.Cu") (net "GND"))
 (segment (start 136.925 78.77) (end 136.925 69.62) (width 0.2) (layer "F.Cu") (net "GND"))
 (segment (start 157.48 43.18) (end 152.4 38.1) (width 0.2) (layer "F.Cu") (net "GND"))
 (segment (start 198.12 43.18) (end 198.12 50.8) (width 0.2) (layer "F.Cu") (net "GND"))
 (segment (start 176.7575 83.085) (end 170.9425 88.9) (width 0.2) (layer "F.Cu") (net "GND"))
 (segment (start 192.305 83.085) (end 178.085 83.085) (width 0.2) (layer "F.Cu") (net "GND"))
 (segment (start 198.12 88.9) (end 192.305 83.085) (width 0.2) (layer "F.Cu") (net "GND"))
 (segment (start 190.5 38.1) (end 193.04 38.1) (width 0.2) (layer "F.Cu") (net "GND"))
 (via (at 140.925 83.82) (size 0.6) (drill 0.3) (layers "F.Cu" "B.Cu") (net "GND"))
 (via (at 190.5 35.56) (size 0.6) (drill 0.3) (layers "F.Cu" "B.Cu") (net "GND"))
 (via (at 139.7 83.82) (size 0.6) (drill 0.3) (layers "F.Cu" "B.Cu") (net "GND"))
 (via (at 185.42 35.56) (size 0.6) (drill 0.3) (layers "F.Cu" "B.Cu") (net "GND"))
 (segment (start 140.925 83.82) (end 139.7 83.82) (width 0.2) (layer "B.Cu") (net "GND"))
 (segment (start 185.42 35.56) (end 190.5 35.56) (width 0.2) (layer "B.Cu") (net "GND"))
 (segment (start 147.32 43.18) (end 147.32 38.1) (width 0.2) (layer "F.Cu") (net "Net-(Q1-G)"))
 (segment (start 147.32 43.18) (end 152.4 43.18) (width 0.2) (layer "F.Cu") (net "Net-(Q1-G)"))
 (segment (start 187.96 27.7625) (end 187.96 38.1) (width 0.2) (layer "F.Cu") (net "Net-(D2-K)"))
 (segment (start 185.425 25.2275) (end 187.96 27.7625) (width 0.2) (layer "F.Cu") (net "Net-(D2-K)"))
 (segment (start 187.96 50.8) (end 187.96 44.45) (width 0.2) (layer "F.Cu") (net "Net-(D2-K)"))
 (segment (start 187.96 41.91) (end 187.96 38.1) (width 0.2) (layer "F.Cu") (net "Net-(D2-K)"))
 (via (at 187.96 44.45) (size 0.6) (drill 0.3) (layers "F.Cu" "B.Cu") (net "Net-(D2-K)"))
 (via (at 187.96 41.91) (size 0.6) (drill 0.3) (layers "F.Cu" "B.Cu") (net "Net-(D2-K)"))
 (segment (start 187.96 44.45) (end 187.96 41.91) (width 0.2) (layer "B.Cu") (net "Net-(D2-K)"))
 (segment (start 170.18 38.1) (end 170.18 45.72) (width 0.2) (layer "F.Cu") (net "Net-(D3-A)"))
 (segment (start 198.12 93.98) (end 196.25 95.85) (width 0.2) (layer "F.Cu") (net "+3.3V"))
 (segment (start 191.77 94.828529) (end 191.77 88.9) (width 0.2) (layer "F.Cu") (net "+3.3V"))
 (segment (start 157.555 84.355) (end 160.585 84.355) (width 0.2) (layer "F.Cu") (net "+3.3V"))
 (segment (start 161.73647 84.355) (end 160.585 84.355) (width 0.2) (layer "F.Cu") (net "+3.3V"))
 (segment (start 146.71 88.9) (end 153.01 88.9) (width 0.2) (layer "F.Cu") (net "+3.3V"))
 (segment (start 192.791471 95.85) (end 191.77 94.828529) (width 0.2) (layer "F.Cu") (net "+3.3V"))
 (segment (start 162.515735 85.134265) (end 161.73647 84.355) (width 0.2) (layer "F.Cu") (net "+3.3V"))
 (segment (start 153.01 88.9) (end 157.555 84.355) (width 0.2) (layer "F.Cu") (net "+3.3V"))
 (segment (start 196.25 95.85) (end 192.791471 95.85) (width 0.2) (layer "F.Cu") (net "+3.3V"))
 (via (at 191.77 88.9) (size 0.6) (drill 0.3) (layers "F.Cu" "B.Cu") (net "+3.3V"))
 (via (at 162.515735 85.134265) (size 0.6) (drill 0.3) (layers "F.Cu" "B.Cu") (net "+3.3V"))
 (segment (start 191.77 88.9) (end 188.004265 85.134265) (width 0.2) (layer "B.Cu") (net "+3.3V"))
 (segment (start 188.004265 85.134265) (end 162.515735 85.134265) (width 0.2) (layer "B.Cu") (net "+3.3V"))
 (segment (start 162.56 90.17) (end 161.825 89.435) (width 0.2) (layer "F.Cu") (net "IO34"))
 (segment (start 161.825 89.435) (end 160.585 89.435) (width 0.2) (layer "F.Cu") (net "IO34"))
 (segment (start 200.66 91.44) (end 194.31 91.44) (width 0.2) (layer "F.Cu") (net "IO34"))
 (via (at 162.56 90.17) (size 0.6) (drill 0.3) (layers "F.Cu" "B.Cu") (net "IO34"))
 (via (at 194.31 91.44) (size 0.6) (drill 0.3) (layers "F.Cu" "B.Cu") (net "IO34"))
 (segment (start 194.31 91.44) (end 193.04 92.71) (width 0.2) (layer "B.Cu") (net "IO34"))
 (segment (start 193.04 92.71) (end 165.1 92.71) (width 0.2) (layer "B.Cu") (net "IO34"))
 (segment (start 165.1 92.71) (end 162.56 90.17) (width 0.2) (layer "B.Cu") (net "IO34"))
 (segment (start 144.78 61.008578) (end 144.78 82.55) (width 0.2) (layer "F.Cu") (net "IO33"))
 (segment (start 144.78 92.71) (end 145.315 93.245) (width 0.2) (layer "F.Cu") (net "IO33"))
 (segment (start 160.485 60.495) (end 145.293578 60.495) (width 0.2) (layer "F.Cu") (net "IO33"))
 (segment (start 145.293578 60.495) (end 144.78 61.008578) (width 0.2) (layer "F.Cu") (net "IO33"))
 (segment (start 145.315 93.245) (end 160.585 93.245) (width 0.2) (layer "F.Cu") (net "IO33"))
 (segment (start 170.18 50.8) (end 160.485 60.495) (width 0.2) (layer "F.Cu") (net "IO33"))
 (via (at 144.78 92.71) (size 0.6) (drill 0.3) (layers "F.Cu" "B.Cu") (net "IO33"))
 (via (at 144.78 82.55) (size 0.6) (drill 0.3) (layers "F.Cu" "B.Cu") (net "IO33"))
 (segment (start 144.78 82.55) (end 144.78 92.71) (width 0.2) (layer "B.Cu") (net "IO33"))
 (segment (start 143.51 63.5) (end 143.51 82.55) (width 0.2) (layer "F.Cu") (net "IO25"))
 (segment (start 142.24 62.23) (end 143.51 63.5) (width 0.2) (layer "F.Cu") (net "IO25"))
 (segment (start 142.24 43.18) (end 142.24 62.23) (width 0.2) (layer "F.Cu") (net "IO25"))
 (segment (start 145.315 94.515) (end 160.585 94.515) (width 0.2) (layer "F.Cu") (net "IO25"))
 (segment (start 143.51 92.71) (end 145.315 94.515) (width 0.2) (layer "F.Cu") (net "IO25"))
 (via (at 143.51 82.55) (size 0.6) (drill 0.3) (layers "F.Cu" "B.Cu") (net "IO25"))
 (via (at 143.51 92.71) (size 0.6) (drill 0.3) (layers "F.Cu" "B.Cu") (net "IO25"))
 (segment (start 143.51 82.55) (end 143.51 92.71) (width 0.2) (layer "B.Cu") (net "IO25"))
 (segment (start 176.244365 43.18) (end 159.329365 60.095) (width 0.2) (layer "F.Cu") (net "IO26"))
 (segment (start 144.78 95.25) (end 145.315 95.785) (width 0.2) (layer "F.Cu") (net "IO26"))
 (segment (start 145.315 95.785) (end 160.585 95.785) (width 0.2) (layer "F.Cu") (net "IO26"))
 (segment (start 144.145002 61.07789) (end 144.145002 82.063402) (width 0.2) (layer "F.Cu") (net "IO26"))
 (segment (start 145.127892 60.095) (end 144.145002 61.07789) (width 0.2) (layer "F.Cu") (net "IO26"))
 (segment (start 159.329365 60.095) (end 145.127892 60.095) (width 0.2) (layer "F.Cu") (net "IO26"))
 (segment (start 180.34 43.18) (end 176.244365 43.18) (width 0.2) (layer "F.Cu") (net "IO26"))
 (via (at 144.78 95.25) (size 0.6) (drill 0.3) (layers "F.Cu" "B.Cu") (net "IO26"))
 (via (at 144.145002 82.063402) (size 0.6) (drill 0.3) (layers "F.Cu" "B.Cu") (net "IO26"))
 (segment (start 144.145002 82.063402) (end 144.145002 94.615002) (width 0.2) (layer "B.Cu") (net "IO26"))
 (segment (start 144.145002 94.615002) (end 144.78 95.25) (width 0.2) (layer "B.Cu") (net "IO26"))
 (segment (start 185.42 38.1) (end 185.42 43.18) (width 0.2) (layer "F.Cu") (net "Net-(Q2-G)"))
 (segment (start 193.04 43.18) (end 185.42 43.18) (width 0.2) (layer "F.Cu") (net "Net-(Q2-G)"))
 (segment (start 142.24 88.9) (end 144.54 91.2) (width 0.2) (layer "F.Cu") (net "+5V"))
 (segment (start 144.54 91.2) (end 146.71 91.2) (width 0.2) (layer "F.Cu") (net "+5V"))
 (segment (start 135.225 78.77) (end 135.225 81.72) (width 0.2) (layer "F.Cu") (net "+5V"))
 (segment (start 135.225 81.72) (end 136.325 82.82) (width 0.2) (layer "F.Cu") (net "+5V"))
 (via (at 136.325 82.82) (size 0.6) (drill 0.3) (layers "F.Cu" "B.Cu") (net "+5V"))
 (via (at 142.24 88.9) (size 0.6) (drill 0.3) (layers "F.Cu" "B.Cu") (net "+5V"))
 (segment (start 142.24 88.735) (end 142.24 88.9) (width 0.2) (layer "B.Cu") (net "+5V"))
 (segment (start 136.325 82.82) (end 142.24 88.735) (width 0.2) (layer "B.Cu") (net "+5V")))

